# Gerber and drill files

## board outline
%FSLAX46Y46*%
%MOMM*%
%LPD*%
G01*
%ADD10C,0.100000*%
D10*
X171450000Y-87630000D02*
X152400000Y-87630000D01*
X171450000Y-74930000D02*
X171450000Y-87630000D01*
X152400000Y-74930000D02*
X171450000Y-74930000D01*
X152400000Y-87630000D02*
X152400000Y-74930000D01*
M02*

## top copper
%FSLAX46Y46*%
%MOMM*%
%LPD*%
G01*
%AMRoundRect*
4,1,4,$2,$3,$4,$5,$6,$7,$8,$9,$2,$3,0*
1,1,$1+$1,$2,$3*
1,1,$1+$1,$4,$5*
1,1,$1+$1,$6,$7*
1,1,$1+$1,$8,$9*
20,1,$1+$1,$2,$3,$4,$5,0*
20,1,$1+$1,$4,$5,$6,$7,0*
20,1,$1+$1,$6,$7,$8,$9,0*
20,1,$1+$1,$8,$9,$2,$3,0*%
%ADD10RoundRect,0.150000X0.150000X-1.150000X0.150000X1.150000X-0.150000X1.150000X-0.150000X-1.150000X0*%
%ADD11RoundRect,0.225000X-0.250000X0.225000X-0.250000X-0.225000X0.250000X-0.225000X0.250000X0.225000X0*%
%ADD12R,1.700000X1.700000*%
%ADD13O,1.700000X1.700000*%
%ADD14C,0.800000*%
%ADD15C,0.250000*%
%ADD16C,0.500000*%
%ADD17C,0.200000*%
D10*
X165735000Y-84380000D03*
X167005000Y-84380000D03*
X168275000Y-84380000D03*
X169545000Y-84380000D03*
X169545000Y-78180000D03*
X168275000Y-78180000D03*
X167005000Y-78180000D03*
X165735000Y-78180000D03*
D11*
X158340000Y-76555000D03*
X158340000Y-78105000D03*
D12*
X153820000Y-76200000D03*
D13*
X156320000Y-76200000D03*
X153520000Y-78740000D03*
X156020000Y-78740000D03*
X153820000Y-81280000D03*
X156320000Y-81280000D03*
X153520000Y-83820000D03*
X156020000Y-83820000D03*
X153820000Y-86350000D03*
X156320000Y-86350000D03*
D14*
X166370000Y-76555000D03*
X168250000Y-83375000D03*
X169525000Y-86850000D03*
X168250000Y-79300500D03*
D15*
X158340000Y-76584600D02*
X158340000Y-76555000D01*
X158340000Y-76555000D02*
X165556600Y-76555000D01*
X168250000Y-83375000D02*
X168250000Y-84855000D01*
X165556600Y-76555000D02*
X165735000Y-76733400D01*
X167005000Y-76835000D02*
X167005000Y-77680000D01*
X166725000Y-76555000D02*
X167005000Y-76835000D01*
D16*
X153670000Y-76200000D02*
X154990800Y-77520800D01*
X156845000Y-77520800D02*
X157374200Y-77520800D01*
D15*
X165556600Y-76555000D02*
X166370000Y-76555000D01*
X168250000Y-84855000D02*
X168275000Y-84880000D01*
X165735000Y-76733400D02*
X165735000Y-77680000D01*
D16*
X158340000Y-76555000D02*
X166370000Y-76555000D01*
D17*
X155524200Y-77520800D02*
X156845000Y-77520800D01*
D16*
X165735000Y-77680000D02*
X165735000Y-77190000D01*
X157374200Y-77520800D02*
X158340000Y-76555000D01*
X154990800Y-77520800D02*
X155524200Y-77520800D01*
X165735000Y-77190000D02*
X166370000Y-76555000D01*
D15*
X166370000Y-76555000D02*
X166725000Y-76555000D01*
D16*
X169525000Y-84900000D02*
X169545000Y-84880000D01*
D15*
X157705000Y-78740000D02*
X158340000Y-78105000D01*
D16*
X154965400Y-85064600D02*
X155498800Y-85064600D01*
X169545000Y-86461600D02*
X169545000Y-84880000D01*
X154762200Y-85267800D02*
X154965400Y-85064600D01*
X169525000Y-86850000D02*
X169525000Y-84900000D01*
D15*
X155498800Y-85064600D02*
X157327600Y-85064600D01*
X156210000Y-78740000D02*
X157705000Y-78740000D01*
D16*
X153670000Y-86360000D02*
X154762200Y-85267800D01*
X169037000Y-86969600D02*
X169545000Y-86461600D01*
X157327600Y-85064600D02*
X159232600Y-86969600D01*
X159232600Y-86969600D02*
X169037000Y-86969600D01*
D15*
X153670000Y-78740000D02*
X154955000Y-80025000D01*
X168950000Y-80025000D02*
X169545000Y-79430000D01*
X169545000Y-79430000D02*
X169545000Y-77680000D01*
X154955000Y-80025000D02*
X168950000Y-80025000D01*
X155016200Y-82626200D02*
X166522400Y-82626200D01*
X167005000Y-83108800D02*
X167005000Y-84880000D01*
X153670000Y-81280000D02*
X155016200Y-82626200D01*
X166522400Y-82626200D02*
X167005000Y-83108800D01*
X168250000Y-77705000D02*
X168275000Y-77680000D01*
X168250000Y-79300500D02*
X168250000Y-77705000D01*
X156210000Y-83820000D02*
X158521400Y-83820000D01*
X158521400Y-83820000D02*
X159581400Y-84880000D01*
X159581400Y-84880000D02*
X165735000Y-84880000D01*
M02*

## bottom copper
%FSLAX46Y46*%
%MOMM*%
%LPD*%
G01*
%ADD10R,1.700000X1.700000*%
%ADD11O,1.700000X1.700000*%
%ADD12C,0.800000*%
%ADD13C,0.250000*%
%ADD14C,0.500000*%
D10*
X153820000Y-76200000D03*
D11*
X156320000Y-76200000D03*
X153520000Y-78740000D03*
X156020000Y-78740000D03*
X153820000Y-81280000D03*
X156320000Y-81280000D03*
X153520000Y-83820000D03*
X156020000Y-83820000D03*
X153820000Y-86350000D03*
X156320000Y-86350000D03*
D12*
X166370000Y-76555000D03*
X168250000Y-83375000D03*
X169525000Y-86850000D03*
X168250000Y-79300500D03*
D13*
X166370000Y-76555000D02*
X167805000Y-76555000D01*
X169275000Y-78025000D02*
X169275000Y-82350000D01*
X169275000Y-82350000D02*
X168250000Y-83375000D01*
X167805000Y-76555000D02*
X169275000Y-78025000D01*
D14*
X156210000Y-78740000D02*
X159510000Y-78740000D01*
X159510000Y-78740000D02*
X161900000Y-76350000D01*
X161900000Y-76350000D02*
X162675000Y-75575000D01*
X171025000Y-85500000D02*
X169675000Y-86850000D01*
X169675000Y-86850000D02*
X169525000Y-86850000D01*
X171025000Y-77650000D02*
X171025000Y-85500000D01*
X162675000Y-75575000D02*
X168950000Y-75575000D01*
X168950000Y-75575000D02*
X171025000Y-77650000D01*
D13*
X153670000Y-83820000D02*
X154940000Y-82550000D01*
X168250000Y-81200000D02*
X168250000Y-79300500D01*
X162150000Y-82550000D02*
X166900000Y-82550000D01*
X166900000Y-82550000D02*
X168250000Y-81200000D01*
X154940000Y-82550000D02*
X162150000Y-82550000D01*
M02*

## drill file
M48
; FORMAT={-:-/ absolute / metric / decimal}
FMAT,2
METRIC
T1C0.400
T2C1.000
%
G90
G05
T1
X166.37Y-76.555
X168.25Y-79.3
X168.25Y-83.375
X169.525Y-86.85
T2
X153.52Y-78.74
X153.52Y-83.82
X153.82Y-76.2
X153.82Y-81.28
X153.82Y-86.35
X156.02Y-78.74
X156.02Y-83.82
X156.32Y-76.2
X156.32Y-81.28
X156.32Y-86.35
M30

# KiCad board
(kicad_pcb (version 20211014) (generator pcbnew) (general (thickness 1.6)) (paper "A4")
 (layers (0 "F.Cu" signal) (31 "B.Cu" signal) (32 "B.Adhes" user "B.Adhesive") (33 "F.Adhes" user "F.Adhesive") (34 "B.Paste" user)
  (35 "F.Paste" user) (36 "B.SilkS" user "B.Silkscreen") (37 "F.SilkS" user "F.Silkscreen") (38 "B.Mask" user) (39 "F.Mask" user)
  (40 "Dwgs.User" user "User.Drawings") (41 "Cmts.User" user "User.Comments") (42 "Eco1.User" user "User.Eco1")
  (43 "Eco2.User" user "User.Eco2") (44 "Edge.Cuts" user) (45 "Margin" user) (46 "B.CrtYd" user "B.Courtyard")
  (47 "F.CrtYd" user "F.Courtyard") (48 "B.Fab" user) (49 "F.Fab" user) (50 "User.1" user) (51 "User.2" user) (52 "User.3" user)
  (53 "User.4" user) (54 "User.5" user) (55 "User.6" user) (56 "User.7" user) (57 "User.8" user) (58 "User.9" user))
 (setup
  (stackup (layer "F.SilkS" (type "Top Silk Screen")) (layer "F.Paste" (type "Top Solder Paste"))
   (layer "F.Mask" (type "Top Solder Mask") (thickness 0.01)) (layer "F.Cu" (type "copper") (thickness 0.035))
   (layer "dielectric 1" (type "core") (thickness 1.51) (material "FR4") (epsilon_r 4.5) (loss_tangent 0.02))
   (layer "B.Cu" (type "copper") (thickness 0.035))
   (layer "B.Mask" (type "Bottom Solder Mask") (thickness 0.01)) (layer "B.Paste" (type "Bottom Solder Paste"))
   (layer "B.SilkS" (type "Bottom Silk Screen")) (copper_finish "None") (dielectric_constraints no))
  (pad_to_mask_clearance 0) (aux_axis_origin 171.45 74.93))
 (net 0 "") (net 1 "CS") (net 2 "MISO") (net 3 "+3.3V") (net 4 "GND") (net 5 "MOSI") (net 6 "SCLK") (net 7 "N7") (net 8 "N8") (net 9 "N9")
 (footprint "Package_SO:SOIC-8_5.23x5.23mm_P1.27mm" (layer "F.Cu") (at 167.64 81.28 90)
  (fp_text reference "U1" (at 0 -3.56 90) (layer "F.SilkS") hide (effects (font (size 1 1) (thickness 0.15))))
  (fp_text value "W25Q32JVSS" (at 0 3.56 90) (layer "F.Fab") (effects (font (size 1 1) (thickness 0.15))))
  (pad "1" smd roundrect (at -3.1 -1.905 90) (size 2.6 0.6) (layers "F.Cu" "F.Paste" "F.Mask") (roundrect_rratio 0.25) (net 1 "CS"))
  (pad "2" smd roundrect (at -3.1 -0.635 90) (size 2.6 0.6) (layers "F.Cu" "F.Paste" "F.Mask") (roundrect_rratio 0.25) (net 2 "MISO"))
  (pad "3" smd roundrect (at -3.1 0.635 90) (size 2.6 0.6) (layers "F.Cu" "F.Paste" "F.Mask") (roundrect_rratio 0.25) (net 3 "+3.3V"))
  (pad "4" smd roundrect (at -3.1 1.905 90) (size 2.6 0.6) (layers "F.Cu" "F.Paste" "F.Mask") (roundrect_rratio 0.25) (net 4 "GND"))
  (pad "5" smd roundrect (at 3.1 1.905 90) (size 2.6 0.6) (layers "F.Cu" "F.Paste" "F.Mask") (roundrect_rratio 0.25) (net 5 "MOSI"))
  (pad "6" smd roundrect (at 3.1 0.635 90) (size 2.6 0.6) (layers "F.Cu" "F.Paste" "F.Mask") (roundrect_rratio 0.25) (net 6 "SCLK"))
  (pad "7" smd roundrect (at 3.1 -0.635 90) (size 2.6 0.6) (layers "F.Cu" "F.Paste" "F.Mask") (roundrect_rratio 0.25) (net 3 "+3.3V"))
  (pad "8" smd roundrect (at 3.1 -1.905 90) (size 2.6 0.6) (layers "F.Cu" "F.Paste" "F.Mask") (roundrect_rratio 0.25) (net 3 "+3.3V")))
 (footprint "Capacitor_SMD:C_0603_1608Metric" (layer "F.Cu") (at 158.34 77.33 -90)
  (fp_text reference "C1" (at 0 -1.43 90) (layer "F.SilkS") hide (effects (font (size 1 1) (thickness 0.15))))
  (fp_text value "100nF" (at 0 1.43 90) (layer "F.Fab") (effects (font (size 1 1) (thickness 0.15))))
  (pad "1" smd roundrect (at -0.775 0 270) (size 0.9 0.95) (layers "F.Cu" "F.Paste" "F.Mask") (roundrect_rratio 0.25) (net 3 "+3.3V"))
  (pad "2" smd roundrect (at 0.775 0 270) (size 0.9 0.95) (layers "F.Cu" "F.Paste" "F.Mask") (roundrect_rratio 0.25) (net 4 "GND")))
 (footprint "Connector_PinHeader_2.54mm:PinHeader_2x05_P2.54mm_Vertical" (layer "F.Cu") (at 153.67 76.2)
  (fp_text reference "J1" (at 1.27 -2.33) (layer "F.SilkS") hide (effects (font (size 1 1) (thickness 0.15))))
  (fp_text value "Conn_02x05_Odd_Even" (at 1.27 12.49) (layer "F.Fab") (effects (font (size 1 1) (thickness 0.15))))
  (pad "1" thru_hole rect (at 0.15 0) (size 1.7 1.7) (drill 1) (layers *.Cu *.Mask) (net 3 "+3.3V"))
  (pad "2" thru_hole oval (at 2.65 0) (size 1.7 1.7) (drill 1) (layers *.Cu *.Mask) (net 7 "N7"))
  (pad "3" thru_hole oval (at -0.15 2.54) (size 1.7 1.7) (drill 1) (layers *.Cu *.Mask) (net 5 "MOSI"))
  (pad "4" thru_hole oval (at 2.35 2.54) (size 1.7 1.7) (drill 1) (layers *.Cu *.Mask) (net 4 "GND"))
  (pad "5" thru_hole oval (at 0.15 5.08) (size 1.7 1.7) (drill 1) (layers *.Cu *.Mask) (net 2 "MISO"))
  (pad "6" thru_hole oval (at 2.65 5.08) (size 1.7 1.7) (drill 1) (layers *.Cu *.Mask) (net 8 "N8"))
  (pad "7" thru_hole oval (at -0.15 7.62) (size 1.7 1.7) (drill 1) (layers *.Cu *.Mask) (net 6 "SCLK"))
  (pad "8" thru_hole oval (at 2.35 7.62) (size 1.7 1.7) (drill 1) (layers *.Cu *.Mask) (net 1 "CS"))
  (pad "9" thru_hole oval (at 0.15 10.15) (size 1.7 1.7) (drill 1) (layers *.Cu *.Mask) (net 4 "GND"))
  (pad "10" thru_hole oval (at 2.65 10.15) (size 1.7 1.7) (drill 1) (layers *.Cu *.Mask) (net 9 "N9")))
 (gr_line (start 171.45 87.63) (end 152.4 87.63) (layer "Edge.Cuts") (width 0.1))
 (gr_line (start 171.45 74.93) (end 171.45 87.63) (layer "Edge.Cuts") (width 0.1))
 (gr_line (start 152.4 74.93) (end 171.45 74.93) (layer "Edge.Cuts") (width 0.1))
 (gr_line (start 152.4 87.63) (end 152.4 74.93) (layer "Edge.Cuts") (width 0.1))
 (segment (start 158.34 76.5846) (end 158.34 76.555) (width 0.25) (layer "F.Cu") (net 3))
 (segment (start 158.34 76.555) (end 165.5566 76.555) (width 0.25) (layer "F.Cu") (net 3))
 (segment (start 168.25 83.375) (end 168.25 84.855) (width 0.25) (layer "F.Cu") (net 3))
 (segment (start 165.5566 76.555) (end 165.735 76.7334) (width 0.25) (layer "F.Cu") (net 3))
 (segment (start 167.005 76.835) (end 167.005 77.68) (width 0.25) (layer "F.Cu") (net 3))
 (segment (start 166.725 76.555) (end 167.005 76.835) (width 0.25) (layer "F.Cu") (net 3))
 (segment (start 153.67 76.2) (end 154.9908 77.5208) (width 0.5) (layer "F.Cu") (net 3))
 (segment (start 156.845 77.5208) (end 157.3742 77.5208) (width 0.5) (layer "F.Cu") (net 3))
 (segment (start 165.5566 76.555) (end 166.37 76.555) (width 0.25) (layer "F.Cu") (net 3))
 (segment (start 168.25 84.855) (end 168.275 84.88) (width 0.25) (layer "F.Cu") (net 3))
 (segment (start 165.735 76.7334) (end 165.735 77.68) (width 0.25) (layer "F.Cu") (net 3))
 (segment (start 158.34 76.555) (end 166.37 76.555) (width 0.5) (layer "F.Cu") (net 3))
 (segment (start 155.5242 77.5208) (end 156.845 77.5208) (width 0.2) (layer "F.Cu") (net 3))
 (segment (start 165.735 77.68) (end 165.735 77.19) (width 0.5) (layer "F.Cu") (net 3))
 (segment (start 157.3742 77.5208) (end 158.34 76.555) (width 0.5) (layer "F.Cu") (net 3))
 (segment (start 154.9908 77.5208) (end 155.5242 77.5208) (width 0.5) (layer "F.Cu") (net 3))
 (segment (start 165.735 77.19) (end 166.37 76.555) (width 0.5) (layer "F.Cu") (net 3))
 (segment (start 166.37 76.555) (end 166.725 76.555) (width 0.25) (layer "F.Cu") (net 3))
 (via (at 166.37 76.555) (size 0.8) (drill 0.4) (layers "F.Cu" "B.Cu") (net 3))
 (via (at 168.25 83.375) (size 0.8) (drill 0.4) (layers "F.Cu" "B.Cu") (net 3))
 (segment (start 166.37 76.555) (end 167.805 76.555) (width 0.25) (layer "B.Cu") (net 3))
 (segment (start 169.275 78.025) (end 169.275 82.35) (width 0.25) (layer "B.Cu") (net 3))
 (segment (start 169.275 82.35) (end 168.25 83.375) (width 0.25) (layer "B.Cu") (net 3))
 (segment (start 167.805 76.555) (end 169.275 78.025) (width 0.25) (layer "B.Cu") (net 3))
 (segment (start 169.525 84.9) (end 169.545 84.88) (width 0.5) (layer "F.Cu") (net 4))
 (segment (start 157.705 78.74) (end 158.34 78.105) (width 0.25) (layer "F.Cu") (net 4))
 (segment (start 154.9654 85.0646) (end 155.4988 85.0646) (width 0.5) (layer "F.Cu") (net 4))
 (segment (start 169.545 86.4616) (end 169.545 84.88) (width 0.5) (layer "F.Cu") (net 4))
 (segment (start 154.7622 85.2678) (end 154.9654 85.0646) (width 0.5) (layer "F.Cu") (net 4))
 (segment (start 169.525 86.85) (end 169.525 84.9) (width 0.5) (layer "F.Cu") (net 4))
 (segment (start 155.4988 85.0646) (end 157.3276 85.0646) (width 0.25) (layer "F.Cu") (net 4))
 (segment (start 156.21 78.74) (end 157.705 78.74) (width 0.25) (layer "F.Cu") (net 4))
 (segment (start 153.67 86.36) (end 154.7622 85.2678) (width 0.5) (layer "F.Cu") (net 4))
 (segment (start 169.037 86.9696) (end 169.545 86.4616) (width 0.5) (layer "F.Cu") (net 4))
 (segment (start 157.3276 85.0646) (end 159.2326 86.9696) (width 0.5) (layer "F.Cu") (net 4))
 (segment (start 159.2326 86.9696) (end 169.037 86.9696) (width 0.5) (layer "F.Cu") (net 4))
 (via (at 169.525 86.85) (size 0.8) (drill 0.4) (layers "F.Cu" "B.Cu") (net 4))
 (segment (start 156.21 78.74) (end 159.51 78.74) (width 0.5) (layer "B.Cu") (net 4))
 (segment (start 159.51 78.74) (end 161.9 76.35) (width 0.5) (layer "B.Cu") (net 4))
 (segment (start 161.9 76.35) (end 162.675 75.575) (width 0.5) (layer "B.Cu") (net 4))
 (segment (start 171.025 85.5) (end 169.675 86.85) (width 0.5) (layer "B.Cu") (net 4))
 (segment (start 169.675 86.85) (end 169.525 86.85) (width 0.5) (layer "B.Cu") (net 4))
 (segment (start 171.025 77.65) (end 171.025 85.5) (width 0.5) (layer "B.Cu") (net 4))
 (segment (start 162.675 75.575) (end 168.95 75.575) (width 0.5) (layer "B.Cu") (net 4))
 (segment (start 168.95 75.575) (end 171.025 77.65) (width 0.5) (layer "B.Cu") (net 4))
 (segment (start 153.67 78.74) (end 154.955 80.025) (width 0.25) (layer "F.Cu") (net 5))
 (segment (start 168.95 80.025) (end 169.545 79.43) (width 0.25) (layer "F.Cu") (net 5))
 (segment (start 169.545 79.43) (end 169.545 77.68) (width 0.25) (layer "F.Cu") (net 5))
 (segment (start 154.955 80.025) (end 168.95 80.025) (width 0.25) (layer "F.Cu") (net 5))
 (segment (start 155.0162 82.6262) (end 166.5224 82.6262) (width 0.25) (layer "F.Cu") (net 2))
 (segment (start 167.005 83.1088) (end 167.005 84.88) (width 0.25) (layer "F.Cu") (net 2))
 (segment (start 153.67 81.28) (end 155.0162 82.6262) (width 0.25) (layer "F.Cu") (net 2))
 (segment (start 166.5224 82.6262) (end 167.005 83.1088) (width 0.25) (layer "F.Cu") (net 2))
 (segment (start 168.25 77.705) (end 168.275 77.68) (width 0.25) (layer "F.Cu") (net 6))
 (segment (start 168.25 79.3005) (end 168.25 77.705) (width 0.25) (layer "F.Cu") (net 6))
 (via (at 168.25 79.3005) (size 0.8) (drill 0.4) (layers "F.Cu" "B.Cu") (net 6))
 (segment (start 153.67 83.82) (end 154.94 82.55) (width 0.25) (layer "B.Cu") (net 6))
 (segment (start 168.25 81.2) (end 168.25 79.3005) (width 0.25) (layer "B.Cu") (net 6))
 (segment (start 162.15 82.55) (end 166.9 82.55) (width 0.25) (layer "B.Cu") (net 6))
 (segment (start 166.9 82.55) (end 168.25 81.2) (width 0.25) (layer "B.Cu") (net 6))
 (segment (start 154.94 82.55) (end 162.15 82.55) (width 0.25) (layer "B.Cu") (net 6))
 (segment (start 156.21 83.82) (end 158.5214 83.82) (width 0.25) (layer "F.Cu") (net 1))
 (segment (start 158.5214 83.82) (end 159.5814 84.88) (width 0.25) (layer "F.Cu") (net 1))
 (segment (start 159.5814 84.88) (end 165.735 84.88) (width 0.25) (layer "F.Cu") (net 1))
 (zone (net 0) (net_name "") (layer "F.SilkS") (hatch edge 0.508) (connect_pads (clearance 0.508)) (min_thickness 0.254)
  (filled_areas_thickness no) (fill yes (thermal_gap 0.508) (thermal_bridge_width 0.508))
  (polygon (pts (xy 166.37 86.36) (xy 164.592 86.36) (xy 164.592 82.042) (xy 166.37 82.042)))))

